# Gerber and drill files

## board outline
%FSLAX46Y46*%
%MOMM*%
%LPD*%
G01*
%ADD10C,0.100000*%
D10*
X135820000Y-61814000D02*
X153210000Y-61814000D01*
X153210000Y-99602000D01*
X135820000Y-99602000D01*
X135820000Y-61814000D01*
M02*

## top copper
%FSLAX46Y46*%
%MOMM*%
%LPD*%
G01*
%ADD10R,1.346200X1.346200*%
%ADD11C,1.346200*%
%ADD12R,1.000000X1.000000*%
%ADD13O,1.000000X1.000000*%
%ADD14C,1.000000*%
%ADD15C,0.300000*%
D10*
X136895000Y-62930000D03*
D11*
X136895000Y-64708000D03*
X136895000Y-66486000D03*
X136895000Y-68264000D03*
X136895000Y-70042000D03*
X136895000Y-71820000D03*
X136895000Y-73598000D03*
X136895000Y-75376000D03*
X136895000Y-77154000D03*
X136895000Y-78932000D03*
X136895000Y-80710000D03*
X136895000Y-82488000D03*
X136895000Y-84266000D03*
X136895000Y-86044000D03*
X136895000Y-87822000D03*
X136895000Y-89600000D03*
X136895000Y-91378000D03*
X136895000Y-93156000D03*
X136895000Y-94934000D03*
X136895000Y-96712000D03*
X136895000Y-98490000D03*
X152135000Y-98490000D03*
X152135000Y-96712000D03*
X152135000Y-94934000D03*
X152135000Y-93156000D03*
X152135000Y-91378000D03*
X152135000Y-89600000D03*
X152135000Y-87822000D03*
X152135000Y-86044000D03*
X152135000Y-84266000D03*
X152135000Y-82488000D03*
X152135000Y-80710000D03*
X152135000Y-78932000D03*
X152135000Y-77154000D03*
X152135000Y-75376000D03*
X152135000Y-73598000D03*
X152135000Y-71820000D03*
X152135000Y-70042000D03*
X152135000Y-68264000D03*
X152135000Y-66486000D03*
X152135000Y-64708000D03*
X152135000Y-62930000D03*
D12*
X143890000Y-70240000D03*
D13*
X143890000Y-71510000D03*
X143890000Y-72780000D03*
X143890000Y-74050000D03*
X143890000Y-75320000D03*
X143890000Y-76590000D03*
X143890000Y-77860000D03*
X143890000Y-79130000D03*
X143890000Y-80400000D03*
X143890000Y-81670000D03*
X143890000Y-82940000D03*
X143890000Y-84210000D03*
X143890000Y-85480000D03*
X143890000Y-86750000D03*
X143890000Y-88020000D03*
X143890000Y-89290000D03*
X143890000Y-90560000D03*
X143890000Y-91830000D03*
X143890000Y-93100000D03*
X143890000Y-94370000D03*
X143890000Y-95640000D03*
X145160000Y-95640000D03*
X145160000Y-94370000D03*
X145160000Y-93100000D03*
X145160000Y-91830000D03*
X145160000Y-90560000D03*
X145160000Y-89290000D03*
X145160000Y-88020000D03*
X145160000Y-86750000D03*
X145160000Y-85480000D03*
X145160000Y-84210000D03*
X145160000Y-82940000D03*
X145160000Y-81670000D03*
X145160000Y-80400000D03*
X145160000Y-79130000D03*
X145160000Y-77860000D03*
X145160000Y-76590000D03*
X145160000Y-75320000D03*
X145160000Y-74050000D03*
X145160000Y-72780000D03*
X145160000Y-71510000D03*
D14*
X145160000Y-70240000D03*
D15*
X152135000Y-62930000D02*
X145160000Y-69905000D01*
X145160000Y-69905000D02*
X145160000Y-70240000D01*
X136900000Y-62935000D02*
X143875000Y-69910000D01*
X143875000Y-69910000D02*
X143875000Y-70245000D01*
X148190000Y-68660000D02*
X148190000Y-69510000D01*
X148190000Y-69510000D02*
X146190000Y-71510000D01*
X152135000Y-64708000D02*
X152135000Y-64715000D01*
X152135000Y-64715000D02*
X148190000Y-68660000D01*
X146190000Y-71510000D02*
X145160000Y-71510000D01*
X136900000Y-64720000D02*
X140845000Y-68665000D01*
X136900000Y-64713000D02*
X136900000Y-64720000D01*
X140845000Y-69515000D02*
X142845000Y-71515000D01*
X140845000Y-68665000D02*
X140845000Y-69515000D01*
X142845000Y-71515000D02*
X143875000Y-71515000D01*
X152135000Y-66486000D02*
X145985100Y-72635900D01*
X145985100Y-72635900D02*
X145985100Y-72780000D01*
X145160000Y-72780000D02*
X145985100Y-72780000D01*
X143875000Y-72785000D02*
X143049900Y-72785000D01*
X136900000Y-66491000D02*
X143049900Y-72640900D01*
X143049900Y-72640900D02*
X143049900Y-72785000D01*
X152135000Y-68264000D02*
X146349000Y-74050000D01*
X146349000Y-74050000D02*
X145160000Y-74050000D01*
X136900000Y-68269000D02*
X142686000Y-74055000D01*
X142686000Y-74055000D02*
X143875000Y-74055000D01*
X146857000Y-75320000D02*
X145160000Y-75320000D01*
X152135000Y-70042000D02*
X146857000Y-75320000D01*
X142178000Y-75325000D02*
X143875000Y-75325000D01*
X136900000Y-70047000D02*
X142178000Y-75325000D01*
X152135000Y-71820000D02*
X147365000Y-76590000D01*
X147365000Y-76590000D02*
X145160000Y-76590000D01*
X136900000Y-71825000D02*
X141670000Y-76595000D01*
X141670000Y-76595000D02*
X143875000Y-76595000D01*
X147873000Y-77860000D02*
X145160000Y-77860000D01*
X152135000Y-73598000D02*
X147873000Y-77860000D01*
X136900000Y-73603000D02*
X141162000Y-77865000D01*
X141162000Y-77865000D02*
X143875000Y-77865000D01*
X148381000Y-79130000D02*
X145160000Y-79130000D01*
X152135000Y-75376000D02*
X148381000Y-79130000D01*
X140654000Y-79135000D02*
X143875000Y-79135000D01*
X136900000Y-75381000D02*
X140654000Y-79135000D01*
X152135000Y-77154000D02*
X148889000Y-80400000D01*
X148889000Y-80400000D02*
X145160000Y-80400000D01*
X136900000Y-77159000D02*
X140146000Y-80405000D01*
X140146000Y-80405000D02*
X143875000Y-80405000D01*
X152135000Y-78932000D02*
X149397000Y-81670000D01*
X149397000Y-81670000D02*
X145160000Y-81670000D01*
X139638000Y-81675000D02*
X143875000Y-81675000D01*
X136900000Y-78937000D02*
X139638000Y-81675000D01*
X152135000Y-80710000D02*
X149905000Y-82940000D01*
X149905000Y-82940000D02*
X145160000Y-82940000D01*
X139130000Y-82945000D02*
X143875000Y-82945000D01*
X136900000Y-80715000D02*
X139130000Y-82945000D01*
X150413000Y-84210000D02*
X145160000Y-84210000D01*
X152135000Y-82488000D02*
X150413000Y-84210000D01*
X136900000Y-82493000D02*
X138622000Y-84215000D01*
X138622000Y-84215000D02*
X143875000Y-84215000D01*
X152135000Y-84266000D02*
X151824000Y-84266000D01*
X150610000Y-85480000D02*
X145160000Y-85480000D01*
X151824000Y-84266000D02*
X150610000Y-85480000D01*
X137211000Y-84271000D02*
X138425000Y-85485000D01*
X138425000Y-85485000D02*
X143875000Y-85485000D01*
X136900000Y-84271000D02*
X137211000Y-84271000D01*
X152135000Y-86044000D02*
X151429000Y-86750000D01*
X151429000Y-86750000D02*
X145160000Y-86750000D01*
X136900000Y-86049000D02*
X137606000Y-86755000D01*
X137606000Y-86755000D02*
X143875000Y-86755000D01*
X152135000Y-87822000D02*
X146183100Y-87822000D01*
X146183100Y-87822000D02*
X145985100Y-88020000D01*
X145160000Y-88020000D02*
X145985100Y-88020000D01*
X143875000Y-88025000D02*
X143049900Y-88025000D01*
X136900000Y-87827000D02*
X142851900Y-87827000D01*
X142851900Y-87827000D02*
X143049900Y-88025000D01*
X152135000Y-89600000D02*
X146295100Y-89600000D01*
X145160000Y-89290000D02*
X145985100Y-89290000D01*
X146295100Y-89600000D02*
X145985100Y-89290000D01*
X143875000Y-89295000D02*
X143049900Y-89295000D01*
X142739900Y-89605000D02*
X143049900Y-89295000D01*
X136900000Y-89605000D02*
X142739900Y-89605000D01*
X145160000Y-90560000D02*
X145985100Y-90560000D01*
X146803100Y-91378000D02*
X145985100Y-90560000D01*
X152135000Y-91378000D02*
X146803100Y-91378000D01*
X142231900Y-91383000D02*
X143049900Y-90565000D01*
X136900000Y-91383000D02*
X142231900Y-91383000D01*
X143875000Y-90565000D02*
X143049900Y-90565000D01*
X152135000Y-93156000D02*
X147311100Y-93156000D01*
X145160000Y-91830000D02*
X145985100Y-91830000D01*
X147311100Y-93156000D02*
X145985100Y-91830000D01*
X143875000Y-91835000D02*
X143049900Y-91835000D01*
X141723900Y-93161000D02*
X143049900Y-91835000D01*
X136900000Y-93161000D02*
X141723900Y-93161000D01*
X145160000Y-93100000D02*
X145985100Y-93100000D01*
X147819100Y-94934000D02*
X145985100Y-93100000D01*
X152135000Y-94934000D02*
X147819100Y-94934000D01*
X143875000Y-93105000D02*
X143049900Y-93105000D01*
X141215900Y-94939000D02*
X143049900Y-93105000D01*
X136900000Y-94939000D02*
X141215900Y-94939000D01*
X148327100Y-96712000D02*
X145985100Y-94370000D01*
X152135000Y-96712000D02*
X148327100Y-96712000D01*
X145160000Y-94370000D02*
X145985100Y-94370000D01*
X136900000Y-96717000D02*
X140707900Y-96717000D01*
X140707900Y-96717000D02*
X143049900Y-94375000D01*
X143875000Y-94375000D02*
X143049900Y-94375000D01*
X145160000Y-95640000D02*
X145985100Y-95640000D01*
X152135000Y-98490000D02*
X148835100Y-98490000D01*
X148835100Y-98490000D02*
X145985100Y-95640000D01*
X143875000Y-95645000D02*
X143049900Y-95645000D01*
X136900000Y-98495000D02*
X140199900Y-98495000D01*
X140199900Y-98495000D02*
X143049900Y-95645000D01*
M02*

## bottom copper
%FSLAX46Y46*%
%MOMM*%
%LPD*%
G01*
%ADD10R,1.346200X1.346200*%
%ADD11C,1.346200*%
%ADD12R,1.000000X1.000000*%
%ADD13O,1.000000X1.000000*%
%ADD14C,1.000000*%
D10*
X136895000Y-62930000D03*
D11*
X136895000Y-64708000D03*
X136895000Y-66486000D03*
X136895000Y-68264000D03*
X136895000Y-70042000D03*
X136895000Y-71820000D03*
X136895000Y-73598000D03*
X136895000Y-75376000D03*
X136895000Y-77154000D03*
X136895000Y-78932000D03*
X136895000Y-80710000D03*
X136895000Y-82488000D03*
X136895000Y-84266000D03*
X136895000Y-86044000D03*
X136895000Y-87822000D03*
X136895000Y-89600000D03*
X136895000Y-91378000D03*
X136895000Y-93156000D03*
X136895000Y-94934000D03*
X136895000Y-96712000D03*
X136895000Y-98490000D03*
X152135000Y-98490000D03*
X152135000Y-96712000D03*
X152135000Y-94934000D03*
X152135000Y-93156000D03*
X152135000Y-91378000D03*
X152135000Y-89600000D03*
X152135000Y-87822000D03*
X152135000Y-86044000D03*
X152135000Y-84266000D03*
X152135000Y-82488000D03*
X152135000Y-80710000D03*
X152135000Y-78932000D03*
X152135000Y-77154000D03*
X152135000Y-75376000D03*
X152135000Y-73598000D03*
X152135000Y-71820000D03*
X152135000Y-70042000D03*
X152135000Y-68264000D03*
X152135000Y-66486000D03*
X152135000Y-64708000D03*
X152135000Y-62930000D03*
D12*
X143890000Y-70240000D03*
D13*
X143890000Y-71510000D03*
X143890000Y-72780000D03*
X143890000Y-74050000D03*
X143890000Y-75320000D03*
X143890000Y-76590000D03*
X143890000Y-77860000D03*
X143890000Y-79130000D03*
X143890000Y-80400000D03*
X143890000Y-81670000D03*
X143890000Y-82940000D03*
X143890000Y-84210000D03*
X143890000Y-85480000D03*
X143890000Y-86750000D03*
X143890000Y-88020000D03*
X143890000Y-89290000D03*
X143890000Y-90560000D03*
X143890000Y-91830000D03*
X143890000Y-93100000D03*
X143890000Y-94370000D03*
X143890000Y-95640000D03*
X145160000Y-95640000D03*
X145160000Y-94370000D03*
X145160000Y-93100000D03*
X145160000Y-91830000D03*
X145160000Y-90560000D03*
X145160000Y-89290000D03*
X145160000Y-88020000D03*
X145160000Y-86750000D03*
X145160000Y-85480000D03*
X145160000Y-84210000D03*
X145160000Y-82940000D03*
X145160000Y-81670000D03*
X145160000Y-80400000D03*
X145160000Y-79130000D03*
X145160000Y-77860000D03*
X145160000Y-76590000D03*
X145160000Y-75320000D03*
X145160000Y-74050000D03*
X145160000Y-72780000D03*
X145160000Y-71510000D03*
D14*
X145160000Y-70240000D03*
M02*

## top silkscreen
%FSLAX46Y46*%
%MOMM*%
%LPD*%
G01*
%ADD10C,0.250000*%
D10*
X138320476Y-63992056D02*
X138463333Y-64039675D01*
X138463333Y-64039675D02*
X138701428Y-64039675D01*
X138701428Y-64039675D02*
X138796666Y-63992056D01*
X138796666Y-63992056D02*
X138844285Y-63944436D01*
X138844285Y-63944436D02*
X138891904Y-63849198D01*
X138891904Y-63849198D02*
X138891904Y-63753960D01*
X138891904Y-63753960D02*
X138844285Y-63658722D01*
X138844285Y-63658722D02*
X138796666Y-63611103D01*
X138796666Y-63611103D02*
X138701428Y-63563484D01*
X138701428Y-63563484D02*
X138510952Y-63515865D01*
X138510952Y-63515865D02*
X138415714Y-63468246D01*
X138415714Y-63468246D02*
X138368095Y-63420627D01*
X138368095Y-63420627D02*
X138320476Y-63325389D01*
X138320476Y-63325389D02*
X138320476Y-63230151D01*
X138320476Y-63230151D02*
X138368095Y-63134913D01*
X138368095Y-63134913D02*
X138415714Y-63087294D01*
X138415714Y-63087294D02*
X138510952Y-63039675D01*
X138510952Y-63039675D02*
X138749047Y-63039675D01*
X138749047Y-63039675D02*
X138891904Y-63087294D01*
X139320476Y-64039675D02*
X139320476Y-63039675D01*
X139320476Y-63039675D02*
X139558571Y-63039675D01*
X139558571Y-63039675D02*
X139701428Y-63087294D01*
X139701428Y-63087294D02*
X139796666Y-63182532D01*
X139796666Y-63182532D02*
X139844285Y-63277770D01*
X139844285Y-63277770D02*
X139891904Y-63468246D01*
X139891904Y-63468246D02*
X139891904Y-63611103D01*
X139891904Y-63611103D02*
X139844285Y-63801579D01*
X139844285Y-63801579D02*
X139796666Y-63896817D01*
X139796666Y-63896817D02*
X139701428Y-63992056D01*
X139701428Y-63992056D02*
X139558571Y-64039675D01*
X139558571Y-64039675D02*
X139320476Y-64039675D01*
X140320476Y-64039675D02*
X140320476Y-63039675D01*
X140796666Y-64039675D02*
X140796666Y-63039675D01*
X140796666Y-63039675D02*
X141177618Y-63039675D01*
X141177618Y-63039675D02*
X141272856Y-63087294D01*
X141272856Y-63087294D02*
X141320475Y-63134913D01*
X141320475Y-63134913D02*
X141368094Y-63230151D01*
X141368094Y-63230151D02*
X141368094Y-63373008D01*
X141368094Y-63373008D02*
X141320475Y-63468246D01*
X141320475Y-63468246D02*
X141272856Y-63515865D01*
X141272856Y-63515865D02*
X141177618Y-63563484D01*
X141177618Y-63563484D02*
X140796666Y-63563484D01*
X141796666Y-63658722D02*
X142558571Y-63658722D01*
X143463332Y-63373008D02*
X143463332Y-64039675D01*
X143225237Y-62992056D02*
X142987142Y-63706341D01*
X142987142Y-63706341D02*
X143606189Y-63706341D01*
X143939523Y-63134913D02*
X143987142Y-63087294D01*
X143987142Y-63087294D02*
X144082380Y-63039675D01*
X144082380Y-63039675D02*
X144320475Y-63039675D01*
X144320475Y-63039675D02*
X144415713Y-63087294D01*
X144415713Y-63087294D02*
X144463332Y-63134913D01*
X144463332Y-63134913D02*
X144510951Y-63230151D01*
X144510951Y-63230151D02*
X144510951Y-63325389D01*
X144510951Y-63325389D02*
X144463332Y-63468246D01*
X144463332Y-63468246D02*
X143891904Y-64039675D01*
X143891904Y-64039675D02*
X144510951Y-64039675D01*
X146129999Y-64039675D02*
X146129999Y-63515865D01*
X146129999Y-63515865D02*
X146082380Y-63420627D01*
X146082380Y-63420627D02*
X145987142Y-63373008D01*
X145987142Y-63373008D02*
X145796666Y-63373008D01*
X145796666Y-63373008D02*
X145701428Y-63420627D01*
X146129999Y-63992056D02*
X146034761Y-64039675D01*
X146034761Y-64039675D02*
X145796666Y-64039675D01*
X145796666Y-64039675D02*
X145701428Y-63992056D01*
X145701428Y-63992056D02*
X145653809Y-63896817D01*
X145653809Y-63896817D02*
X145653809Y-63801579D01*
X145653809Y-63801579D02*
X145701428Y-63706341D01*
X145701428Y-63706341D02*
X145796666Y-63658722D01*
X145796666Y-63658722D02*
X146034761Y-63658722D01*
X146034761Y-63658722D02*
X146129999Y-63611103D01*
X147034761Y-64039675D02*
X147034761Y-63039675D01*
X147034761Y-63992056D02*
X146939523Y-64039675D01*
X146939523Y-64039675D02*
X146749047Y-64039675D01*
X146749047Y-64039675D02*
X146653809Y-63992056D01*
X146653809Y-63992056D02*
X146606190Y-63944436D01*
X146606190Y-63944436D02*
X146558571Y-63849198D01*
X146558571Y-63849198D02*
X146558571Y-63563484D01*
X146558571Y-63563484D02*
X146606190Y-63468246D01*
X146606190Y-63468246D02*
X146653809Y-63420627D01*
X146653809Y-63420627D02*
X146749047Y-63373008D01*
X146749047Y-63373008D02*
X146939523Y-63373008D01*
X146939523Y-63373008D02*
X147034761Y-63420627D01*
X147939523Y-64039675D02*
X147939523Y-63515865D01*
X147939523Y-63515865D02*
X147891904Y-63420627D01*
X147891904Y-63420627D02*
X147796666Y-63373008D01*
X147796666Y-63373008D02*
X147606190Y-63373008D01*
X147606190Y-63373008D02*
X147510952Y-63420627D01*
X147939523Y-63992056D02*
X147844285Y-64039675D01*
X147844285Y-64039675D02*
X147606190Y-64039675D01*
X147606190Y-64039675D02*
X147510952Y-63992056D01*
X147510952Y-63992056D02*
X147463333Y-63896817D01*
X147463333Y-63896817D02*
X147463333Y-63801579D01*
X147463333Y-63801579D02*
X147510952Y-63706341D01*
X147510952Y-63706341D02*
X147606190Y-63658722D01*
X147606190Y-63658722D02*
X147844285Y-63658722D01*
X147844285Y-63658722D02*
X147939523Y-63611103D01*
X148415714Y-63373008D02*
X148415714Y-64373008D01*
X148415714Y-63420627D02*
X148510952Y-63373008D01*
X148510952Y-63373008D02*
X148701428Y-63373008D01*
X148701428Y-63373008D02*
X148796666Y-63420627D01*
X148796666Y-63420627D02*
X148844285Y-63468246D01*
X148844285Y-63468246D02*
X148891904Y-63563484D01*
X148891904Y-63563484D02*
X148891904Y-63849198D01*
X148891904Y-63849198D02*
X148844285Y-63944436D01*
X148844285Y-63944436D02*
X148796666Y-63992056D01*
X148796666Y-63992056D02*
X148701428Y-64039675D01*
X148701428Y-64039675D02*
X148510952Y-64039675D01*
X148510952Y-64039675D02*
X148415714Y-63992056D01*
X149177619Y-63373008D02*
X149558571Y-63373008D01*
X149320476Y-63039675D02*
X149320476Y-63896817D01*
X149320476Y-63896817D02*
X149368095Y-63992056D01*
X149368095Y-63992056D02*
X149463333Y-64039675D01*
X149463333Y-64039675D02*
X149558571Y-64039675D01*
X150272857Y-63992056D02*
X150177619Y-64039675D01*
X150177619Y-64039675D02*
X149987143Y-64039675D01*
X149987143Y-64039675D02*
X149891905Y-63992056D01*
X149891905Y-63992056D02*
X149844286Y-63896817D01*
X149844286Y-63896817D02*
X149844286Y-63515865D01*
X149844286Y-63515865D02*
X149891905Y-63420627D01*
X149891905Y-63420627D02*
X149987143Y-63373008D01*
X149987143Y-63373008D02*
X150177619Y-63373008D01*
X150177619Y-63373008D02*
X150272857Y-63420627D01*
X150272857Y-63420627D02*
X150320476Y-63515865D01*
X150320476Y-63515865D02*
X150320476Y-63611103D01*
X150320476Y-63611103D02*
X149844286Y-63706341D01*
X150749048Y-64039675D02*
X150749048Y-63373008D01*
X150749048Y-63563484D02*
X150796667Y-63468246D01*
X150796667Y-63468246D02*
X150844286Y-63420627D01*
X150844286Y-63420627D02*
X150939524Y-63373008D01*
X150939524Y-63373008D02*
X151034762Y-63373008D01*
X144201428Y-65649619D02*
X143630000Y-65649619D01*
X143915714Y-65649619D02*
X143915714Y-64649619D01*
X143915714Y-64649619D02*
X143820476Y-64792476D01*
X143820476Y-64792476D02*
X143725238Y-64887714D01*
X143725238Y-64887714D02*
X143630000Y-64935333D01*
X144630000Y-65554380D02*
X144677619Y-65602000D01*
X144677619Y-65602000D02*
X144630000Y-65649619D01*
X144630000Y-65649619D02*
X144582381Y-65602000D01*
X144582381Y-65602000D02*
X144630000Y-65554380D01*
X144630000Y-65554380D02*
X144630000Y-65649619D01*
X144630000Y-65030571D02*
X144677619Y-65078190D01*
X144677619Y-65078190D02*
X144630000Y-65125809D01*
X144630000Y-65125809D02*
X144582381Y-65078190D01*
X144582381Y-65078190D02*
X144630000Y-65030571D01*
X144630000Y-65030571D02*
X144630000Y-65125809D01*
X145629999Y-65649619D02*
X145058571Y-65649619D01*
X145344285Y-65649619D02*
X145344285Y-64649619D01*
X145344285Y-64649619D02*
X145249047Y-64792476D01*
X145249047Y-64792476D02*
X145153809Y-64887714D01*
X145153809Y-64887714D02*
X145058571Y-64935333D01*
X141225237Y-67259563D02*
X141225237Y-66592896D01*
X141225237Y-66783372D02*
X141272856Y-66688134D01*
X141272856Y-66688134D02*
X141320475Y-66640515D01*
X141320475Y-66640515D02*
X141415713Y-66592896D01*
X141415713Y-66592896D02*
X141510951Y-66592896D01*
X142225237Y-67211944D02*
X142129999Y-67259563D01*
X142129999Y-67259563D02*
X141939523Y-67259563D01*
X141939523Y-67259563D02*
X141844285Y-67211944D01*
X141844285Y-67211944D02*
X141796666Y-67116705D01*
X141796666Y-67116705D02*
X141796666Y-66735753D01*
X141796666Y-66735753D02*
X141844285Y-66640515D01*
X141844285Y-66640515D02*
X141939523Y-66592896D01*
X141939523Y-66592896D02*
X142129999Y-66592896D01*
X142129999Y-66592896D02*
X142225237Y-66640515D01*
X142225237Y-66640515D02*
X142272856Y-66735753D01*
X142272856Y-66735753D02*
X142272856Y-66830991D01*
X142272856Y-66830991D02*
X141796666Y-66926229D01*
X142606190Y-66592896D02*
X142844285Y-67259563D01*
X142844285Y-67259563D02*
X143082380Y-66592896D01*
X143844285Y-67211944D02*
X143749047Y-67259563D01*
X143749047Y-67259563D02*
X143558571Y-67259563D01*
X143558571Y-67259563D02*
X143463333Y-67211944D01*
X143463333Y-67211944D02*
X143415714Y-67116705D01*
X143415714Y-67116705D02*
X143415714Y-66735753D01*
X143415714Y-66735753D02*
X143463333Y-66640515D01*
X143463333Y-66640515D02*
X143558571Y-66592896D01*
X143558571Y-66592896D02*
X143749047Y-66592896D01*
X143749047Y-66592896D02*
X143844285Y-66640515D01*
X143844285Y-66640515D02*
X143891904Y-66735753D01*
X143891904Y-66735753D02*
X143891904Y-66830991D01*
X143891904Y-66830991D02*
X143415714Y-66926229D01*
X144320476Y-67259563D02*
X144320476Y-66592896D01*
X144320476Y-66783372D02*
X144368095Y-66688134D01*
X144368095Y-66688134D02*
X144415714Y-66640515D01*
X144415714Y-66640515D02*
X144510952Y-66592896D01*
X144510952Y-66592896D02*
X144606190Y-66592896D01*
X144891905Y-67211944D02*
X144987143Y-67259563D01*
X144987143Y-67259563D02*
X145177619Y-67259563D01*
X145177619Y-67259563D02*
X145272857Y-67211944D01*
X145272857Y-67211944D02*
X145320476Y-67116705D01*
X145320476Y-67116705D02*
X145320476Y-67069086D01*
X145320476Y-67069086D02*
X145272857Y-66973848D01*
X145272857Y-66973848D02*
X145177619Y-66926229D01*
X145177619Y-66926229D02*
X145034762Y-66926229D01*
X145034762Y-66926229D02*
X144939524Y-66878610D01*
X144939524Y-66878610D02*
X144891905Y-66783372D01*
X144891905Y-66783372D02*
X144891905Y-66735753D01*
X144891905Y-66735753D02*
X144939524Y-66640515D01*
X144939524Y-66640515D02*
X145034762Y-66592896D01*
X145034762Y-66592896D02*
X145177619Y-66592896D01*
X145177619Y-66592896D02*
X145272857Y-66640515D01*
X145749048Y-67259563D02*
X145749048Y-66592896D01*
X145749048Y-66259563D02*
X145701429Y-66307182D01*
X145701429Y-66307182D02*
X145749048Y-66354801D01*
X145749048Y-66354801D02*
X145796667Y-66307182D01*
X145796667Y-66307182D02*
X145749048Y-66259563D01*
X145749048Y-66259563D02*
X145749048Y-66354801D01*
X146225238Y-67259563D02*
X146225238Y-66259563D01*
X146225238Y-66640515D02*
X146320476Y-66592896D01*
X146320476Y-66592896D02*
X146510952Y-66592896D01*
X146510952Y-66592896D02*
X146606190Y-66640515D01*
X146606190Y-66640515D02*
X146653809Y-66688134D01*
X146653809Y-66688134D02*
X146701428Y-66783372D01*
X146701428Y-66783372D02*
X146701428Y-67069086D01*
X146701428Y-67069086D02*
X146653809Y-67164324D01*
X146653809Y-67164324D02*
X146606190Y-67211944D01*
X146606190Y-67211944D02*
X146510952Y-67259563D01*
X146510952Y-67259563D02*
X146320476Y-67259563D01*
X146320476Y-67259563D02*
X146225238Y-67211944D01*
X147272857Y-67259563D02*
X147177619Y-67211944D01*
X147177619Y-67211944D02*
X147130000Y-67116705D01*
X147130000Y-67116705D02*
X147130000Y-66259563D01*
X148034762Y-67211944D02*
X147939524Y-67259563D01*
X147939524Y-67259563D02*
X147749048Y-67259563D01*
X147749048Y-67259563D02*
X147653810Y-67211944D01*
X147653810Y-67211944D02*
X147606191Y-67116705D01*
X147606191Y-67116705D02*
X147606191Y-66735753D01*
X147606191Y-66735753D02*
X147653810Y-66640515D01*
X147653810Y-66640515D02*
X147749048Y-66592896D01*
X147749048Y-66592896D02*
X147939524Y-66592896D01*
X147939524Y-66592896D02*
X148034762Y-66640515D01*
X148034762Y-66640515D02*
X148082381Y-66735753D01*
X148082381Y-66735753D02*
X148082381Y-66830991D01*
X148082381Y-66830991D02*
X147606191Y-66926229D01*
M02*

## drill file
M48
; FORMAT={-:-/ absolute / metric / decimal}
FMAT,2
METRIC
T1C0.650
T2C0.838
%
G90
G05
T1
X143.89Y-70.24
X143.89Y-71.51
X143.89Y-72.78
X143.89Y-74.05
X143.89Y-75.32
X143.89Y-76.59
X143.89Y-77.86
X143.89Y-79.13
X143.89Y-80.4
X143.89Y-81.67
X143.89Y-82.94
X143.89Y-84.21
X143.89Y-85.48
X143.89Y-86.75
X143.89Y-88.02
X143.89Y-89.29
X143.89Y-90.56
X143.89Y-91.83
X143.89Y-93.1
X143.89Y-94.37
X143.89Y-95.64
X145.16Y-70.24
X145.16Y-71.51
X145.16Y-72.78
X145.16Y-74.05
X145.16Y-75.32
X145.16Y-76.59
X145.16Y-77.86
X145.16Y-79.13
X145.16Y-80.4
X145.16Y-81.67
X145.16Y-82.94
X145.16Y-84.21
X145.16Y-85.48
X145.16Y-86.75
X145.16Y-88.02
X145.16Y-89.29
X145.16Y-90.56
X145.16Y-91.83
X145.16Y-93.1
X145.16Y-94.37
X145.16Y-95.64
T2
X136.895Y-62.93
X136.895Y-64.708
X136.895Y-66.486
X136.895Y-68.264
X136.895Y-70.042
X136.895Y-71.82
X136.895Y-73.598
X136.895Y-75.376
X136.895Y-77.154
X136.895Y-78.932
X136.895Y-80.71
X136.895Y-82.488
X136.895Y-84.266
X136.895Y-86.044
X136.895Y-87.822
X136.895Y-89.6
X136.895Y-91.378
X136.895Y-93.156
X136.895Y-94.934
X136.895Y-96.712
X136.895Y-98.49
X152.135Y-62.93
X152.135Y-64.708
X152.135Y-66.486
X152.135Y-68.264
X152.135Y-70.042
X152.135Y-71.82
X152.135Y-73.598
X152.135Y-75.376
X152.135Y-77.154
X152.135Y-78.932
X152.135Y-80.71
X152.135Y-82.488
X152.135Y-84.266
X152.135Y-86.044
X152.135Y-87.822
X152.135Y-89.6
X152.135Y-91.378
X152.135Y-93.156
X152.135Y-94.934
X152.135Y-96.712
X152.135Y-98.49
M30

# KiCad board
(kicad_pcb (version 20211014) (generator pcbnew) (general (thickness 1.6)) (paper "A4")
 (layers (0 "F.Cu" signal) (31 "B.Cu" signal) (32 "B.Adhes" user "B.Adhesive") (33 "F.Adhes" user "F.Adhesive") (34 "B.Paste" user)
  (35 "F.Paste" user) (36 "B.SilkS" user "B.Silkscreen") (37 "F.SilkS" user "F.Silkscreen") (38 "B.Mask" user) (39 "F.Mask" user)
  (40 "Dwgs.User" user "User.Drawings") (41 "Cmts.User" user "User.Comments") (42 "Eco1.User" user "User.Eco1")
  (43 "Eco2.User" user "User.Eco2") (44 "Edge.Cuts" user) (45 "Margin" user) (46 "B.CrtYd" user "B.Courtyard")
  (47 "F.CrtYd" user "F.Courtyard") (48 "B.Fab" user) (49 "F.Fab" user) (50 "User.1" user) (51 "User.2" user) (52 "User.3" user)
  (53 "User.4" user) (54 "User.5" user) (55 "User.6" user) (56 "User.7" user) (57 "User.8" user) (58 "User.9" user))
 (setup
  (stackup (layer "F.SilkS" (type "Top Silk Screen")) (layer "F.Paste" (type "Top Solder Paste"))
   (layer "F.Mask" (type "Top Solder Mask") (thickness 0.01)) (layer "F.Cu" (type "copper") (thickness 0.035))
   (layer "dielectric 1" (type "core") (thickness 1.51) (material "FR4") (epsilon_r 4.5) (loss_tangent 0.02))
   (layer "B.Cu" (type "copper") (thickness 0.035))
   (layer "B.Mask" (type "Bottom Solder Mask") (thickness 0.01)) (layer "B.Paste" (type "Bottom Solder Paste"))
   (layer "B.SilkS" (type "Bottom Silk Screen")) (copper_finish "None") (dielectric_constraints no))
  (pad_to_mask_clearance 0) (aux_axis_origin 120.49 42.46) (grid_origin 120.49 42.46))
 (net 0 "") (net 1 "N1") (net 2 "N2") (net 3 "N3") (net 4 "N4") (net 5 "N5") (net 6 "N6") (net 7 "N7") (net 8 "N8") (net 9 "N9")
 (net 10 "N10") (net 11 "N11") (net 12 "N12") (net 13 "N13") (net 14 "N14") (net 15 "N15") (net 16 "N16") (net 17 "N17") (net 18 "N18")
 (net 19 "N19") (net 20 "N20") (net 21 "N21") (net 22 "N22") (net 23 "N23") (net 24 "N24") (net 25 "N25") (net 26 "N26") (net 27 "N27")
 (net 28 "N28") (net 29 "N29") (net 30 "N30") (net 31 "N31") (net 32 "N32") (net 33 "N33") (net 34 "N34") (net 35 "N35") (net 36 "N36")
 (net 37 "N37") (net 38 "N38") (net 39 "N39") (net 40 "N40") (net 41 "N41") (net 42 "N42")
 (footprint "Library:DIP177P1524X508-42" (layer "F.Cu") (at 152.135 98.49)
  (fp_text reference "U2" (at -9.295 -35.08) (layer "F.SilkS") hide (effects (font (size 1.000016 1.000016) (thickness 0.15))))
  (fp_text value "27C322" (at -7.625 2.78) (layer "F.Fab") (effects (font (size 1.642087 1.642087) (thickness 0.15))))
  (pad "1" thru_hole rect (at -15.24 -35.56) (size 1.3462 1.3462) (drill 0.8382) (layers *.Cu *.Mask) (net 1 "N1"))
  (pad "2" thru_hole circle (at -15.24 -33.782) (size 1.3462 1.3462) (drill 0.8382) (layers *.Cu *.Mask) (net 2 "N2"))
  (pad "3" thru_hole circle (at -15.24 -32.004) (size 1.3462 1.3462) (drill 0.8382) (layers *.Cu *.Mask) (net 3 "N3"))
  (pad "4" thru_hole circle (at -15.24 -30.226) (size 1.3462 1.3462) (drill 0.8382) (layers *.Cu *.Mask) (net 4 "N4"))
  (pad "5" thru_hole circle (at -15.24 -28.448) (size 1.3462 1.3462) (drill 0.8382) (layers *.Cu *.Mask) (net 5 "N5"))
  (pad "6" thru_hole circle (at -15.24 -26.67) (size 1.3462 1.3462) (drill 0.8382) (layers *.Cu *.Mask) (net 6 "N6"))
  (pad "7" thru_hole circle (at -15.24 -24.892) (size 1.3462 1.3462) (drill 0.8382) (layers *.Cu *.Mask) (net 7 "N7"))
  (pad "8" thru_hole circle (at -15.24 -23.114) (size 1.3462 1.3462) (drill 0.8382) (layers *.Cu *.Mask) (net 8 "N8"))
  (pad "9" thru_hole circle (at -15.24 -21.336) (size 1.3462 1.3462) (drill 0.8382) (layers *.Cu *.Mask) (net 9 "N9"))
  (pad "10" thru_hole circle (at -15.24 -19.558) (size 1.3462 1.3462) (drill 0.8382) (layers *.Cu *.Mask) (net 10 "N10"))
  (pad "11" thru_hole circle (at -15.24 -17.78) (size 1.3462 1.3462) (drill 0.8382) (layers *.Cu *.Mask) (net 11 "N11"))
  (pad "12" thru_hole circle (at -15.24 -16.002) (size 1.3462 1.3462) (drill 0.8382) (layers *.Cu *.Mask) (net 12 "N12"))
  (pad "13" thru_hole circle (at -15.24 -14.224) (size 1.3462 1.3462) (drill 0.8382) (layers *.Cu *.Mask) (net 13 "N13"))
  (pad "14" thru_hole circle (at -15.24 -12.446) (size 1.3462 1.3462) (drill 0.8382) (layers *.Cu *.Mask) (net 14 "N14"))
  (pad "15" thru_hole circle (at -15.24 -10.668) (size 1.3462 1.3462) (drill 0.8382) (layers *.Cu *.Mask) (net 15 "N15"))
  (pad "16" thru_hole circle (at -15.24 -8.89) (size 1.3462 1.3462) (drill 0.8382) (layers *.Cu *.Mask) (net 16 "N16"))
  (pad "17" thru_hole circle (at -15.24 -7.112) (size 1.3462 1.3462) (drill 0.8382) (layers *.Cu *.Mask) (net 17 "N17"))
  (pad "18" thru_hole circle (at -15.24 -5.334) (size 1.3462 1.3462) (drill 0.8382) (layers *.Cu *.Mask) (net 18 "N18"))
  (pad "19" thru_hole circle (at -15.24 -3.556) (size 1.3462 1.3462) (drill 0.8382) (layers *.Cu *.Mask) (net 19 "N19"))
  (pad "20" thru_hole circle (at -15.24 -1.778) (size 1.3462 1.3462) (drill 0.8382) (layers *.Cu *.Mask) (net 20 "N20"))
  (pad "21" thru_hole circle (at -15.24 0) (size 1.3462 1.3462) (drill 0.8382) (layers *.Cu *.Mask) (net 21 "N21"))
  (pad "22" thru_hole circle (at 0 0) (size 1.3462 1.3462) (drill 0.8382) (layers *.Cu *.Mask) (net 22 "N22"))
  (pad "23" thru_hole circle (at 0 -1.778) (size 1.3462 1.3462) (drill 0.8382) (layers *.Cu *.Mask) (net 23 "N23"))
  (pad "24" thru_hole circle (at 0 -3.556) (size 1.3462 1.3462) (drill 0.8382) (layers *.Cu *.Mask) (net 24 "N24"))
  (pad "25" thru_hole circle (at 0 -5.334) (size 1.3462 1.3462) (drill 0.8382) (layers *.Cu *.Mask) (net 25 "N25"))
  (pad "26" thru_hole circle (at 0 -7.112) (size 1.3462 1.3462) (drill 0.8382) (layers *.Cu *.Mask) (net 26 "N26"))
  (pad "27" thru_hole circle (at 0 -8.89) (size 1.3462 1.3462) (drill 0.8382) (layers *.Cu *.Mask) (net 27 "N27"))
  (pad "28" thru_hole circle (at 0 -10.668) (size 1.3462 1.3462) (drill 0.8382) (layers *.Cu *.Mask) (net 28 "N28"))
  (pad "29" thru_hole circle (at 0 -12.446) (size 1.3462 1.3462) (drill 0.8382) (layers *.Cu *.Mask) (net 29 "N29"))
  (pad "30" thru_hole circle (at 0 -14.224) (size 1.3462 1.3462) (drill 0.8382) (layers *.Cu *.Mask) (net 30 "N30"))
  (pad "31" thru_hole circle (at 0 -16.002) (size 1.3462 1.3462) (drill 0.8382) (layers *.Cu *.Mask) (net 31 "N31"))
  (pad "32" thru_hole circle (at 0 -17.78) (size 1.3462 1.3462) (drill 0.8382) (layers *.Cu *.Mask) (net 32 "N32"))
  (pad "33" thru_hole circle (at 0 -19.558) (size 1.3462 1.3462) (drill 0.8382) (layers *.Cu *.Mask) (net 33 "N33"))
  (pad "34" thru_hole circle (at 0 -21.336) (size 1.3462 1.3462) (drill 0.8382) (layers *.Cu *.Mask) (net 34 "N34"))
  (pad "35" thru_hole circle (at 0 -23.114) (size 1.3462 1.3462) (drill 0.8382) (layers *.Cu *.Mask) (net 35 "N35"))
  (pad "36" thru_hole circle (at 0 -24.892) (size 1.3462 1.3462) (drill 0.8382) (layers *.Cu *.Mask) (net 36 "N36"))
  (pad "37" thru_hole circle (at 0 -26.67) (size 1.3462 1.3462) (drill 0.8382) (layers *.Cu *.Mask) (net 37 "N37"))
  (pad "38" thru_hole circle (at 0 -28.448) (size 1.3462 1.3462) (drill 0.8382) (layers *.Cu *.Mask) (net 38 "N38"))
  (pad "39" thru_hole circle (at 0 -30.226) (size 1.3462 1.3462) (drill 0.8382) (layers *.Cu *.Mask) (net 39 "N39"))
  (pad "40" thru_hole circle (at 0 -32.004) (size 1.3462 1.3462) (drill 0.8382) (layers *.Cu *.Mask) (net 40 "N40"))
  (pad "41" thru_hole circle (at 0 -33.782) (size 1.3462 1.3462) (drill 0.8382) (layers *.Cu *.Mask) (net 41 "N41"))
  (pad "42" thru_hole circle (at 0 -35.56) (size 1.3462 1.3462) (drill 0.8382) (layers *.Cu *.Mask) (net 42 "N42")))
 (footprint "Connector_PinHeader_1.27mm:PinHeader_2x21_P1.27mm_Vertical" (layer "B.Cu") (at 145.16 70.24 180)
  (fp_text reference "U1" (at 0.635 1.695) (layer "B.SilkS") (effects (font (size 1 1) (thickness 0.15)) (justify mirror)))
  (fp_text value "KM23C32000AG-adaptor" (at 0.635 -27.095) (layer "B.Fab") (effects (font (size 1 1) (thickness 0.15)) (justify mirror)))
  (pad "1" thru_hole rect (at 1.27 0 180) (size 1 1) (drill 0.65) (layers *.Cu *.Mask) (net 1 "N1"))
  (pad "2" thru_hole oval (at 1.27 -1.27 180) (size 1 1) (drill 0.65) (layers *.Cu *.Mask) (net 2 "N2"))
  (pad "3" thru_hole oval (at 1.27 -2.54 180) (size 1 1) (drill 0.65) (layers *.Cu *.Mask) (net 3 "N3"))
  (pad "4" thru_hole oval (at 1.27 -3.81 180) (size 1 1) (drill 0.65) (layers *.Cu *.Mask) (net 4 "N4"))
  (pad "5" thru_hole oval (at 1.27 -5.08 180) (size 1 1) (drill 0.65) (layers *.Cu *.Mask) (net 5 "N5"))
  (pad "6" thru_hole oval (at 1.27 -6.35 180) (size 1 1) (drill 0.65) (layers *.Cu *.Mask) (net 6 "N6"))
  (pad "7" thru_hole oval (at 1.27 -7.62 180) (size 1 1) (drill 0.65) (layers *.Cu *.Mask) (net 7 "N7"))
  (pad "8" thru_hole oval (at 1.27 -8.89 180) (size 1 1) (drill 0.65) (layers *.Cu *.Mask) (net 8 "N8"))
  (pad "9" thru_hole oval (at 1.27 -10.16 180) (size 1 1) (drill 0.65) (layers *.Cu *.Mask) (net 9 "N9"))
  (pad "10" thru_hole oval (at 1.27 -11.43 180) (size 1 1) (drill 0.65) (layers *.Cu *.Mask) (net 10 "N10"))
  (pad "11" thru_hole oval (at 1.27 -12.7 180) (size 1 1) (drill 0.65) (layers *.Cu *.Mask) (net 11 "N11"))
  (pad "12" thru_hole oval (at 1.27 -13.97 180) (size 1 1) (drill 0.65) (layers *.Cu *.Mask) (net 12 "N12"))
  (pad "13" thru_hole oval (at 1.27 -15.24 180) (size 1 1) (drill 0.65) (layers *.Cu *.Mask) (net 13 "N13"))
  (pad "14" thru_hole oval (at 1.27 -16.51 180) (size 1 1) (drill 0.65) (layers *.Cu *.Mask) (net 14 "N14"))
  (pad "15" thru_hole oval (at 1.27 -17.78 180) (size 1 1) (drill 0.65) (layers *.Cu *.Mask) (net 15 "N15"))
  (pad "16" thru_hole oval (at 1.27 -19.05 180) (size 1 1) (drill 0.65) (layers *.Cu *.Mask) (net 16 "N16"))
  (pad "17" thru_hole oval (at 1.27 -20.32 180) (size 1 1) (drill 0.65) (layers *.Cu *.Mask) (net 17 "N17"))
  (pad "18" thru_hole oval (at 1.27 -21.59 180) (size 1 1) (drill 0.65) (layers *.Cu *.Mask) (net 18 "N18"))
  (pad "19" thru_hole oval (at 1.27 -22.86 180) (size 1 1) (drill 0.65) (layers *.Cu *.Mask) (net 19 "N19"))
  (pad "20" thru_hole oval (at 1.27 -24.13 180) (size 1 1) (drill 0.65) (layers *.Cu *.Mask) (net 20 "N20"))
  (pad "21" thru_hole oval (at 1.27 -25.4 180) (size 1 1) (drill 0.65) (layers *.Cu *.Mask) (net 21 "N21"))
  (pad "22" thru_hole oval (at 0 -25.4 180) (size 1 1) (drill 0.65) (layers *.Cu *.Mask) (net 22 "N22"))
  (pad "23" thru_hole oval (at 0 -24.13 180) (size 1 1) (drill 0.65) (layers *.Cu *.Mask) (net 23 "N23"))
  (pad "24" thru_hole oval (at 0 -22.86 180) (size 1 1) (drill 0.65) (layers *.Cu *.Mask) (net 24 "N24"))
  (pad "25" thru_hole oval (at 0 -21.59 180) (size 1 1) (drill 0.65) (layers *.Cu *.Mask) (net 25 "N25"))
  (pad "26" thru_hole oval (at 0 -20.32 180) (size 1 1) (drill 0.65) (layers *.Cu *.Mask) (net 26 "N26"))
  (pad "27" thru_hole oval (at 0 -19.05 180) (size 1 1) (drill 0.65) (layers *.Cu *.Mask) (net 27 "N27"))
  (pad "28" thru_hole oval (at 0 -17.78 180) (size 1 1) (drill 0.65) (layers *.Cu *.Mask) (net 28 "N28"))
  (pad "29" thru_hole oval (at 0 -16.51 180) (size 1 1) (drill 0.65) (layers *.Cu *.Mask) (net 29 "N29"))
  (pad "30" thru_hole oval (at 0 -15.24 180) (size 1 1) (drill 0.65) (layers *.Cu *.Mask) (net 30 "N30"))
  (pad "31" thru_hole oval (at 0 -13.97 180) (size 1 1) (drill 0.65) (layers *.Cu *.Mask) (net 31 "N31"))
  (pad "32" thru_hole oval (at 0 -12.7 180) (size 1 1) (drill 0.65) (layers *.Cu *.Mask) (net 32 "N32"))
  (pad "33" thru_hole oval (at 0 -11.43 180) (size 1 1) (drill 0.65) (layers *.Cu *.Mask) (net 33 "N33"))
  (pad "34" thru_hole oval (at 0 -10.16 180) (size 1 1) (drill 0.65) (layers *.Cu *.Mask) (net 34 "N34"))
  (pad "35" thru_hole oval (at 0 -8.89 180) (size 1 1) (drill 0.65) (layers *.Cu *.Mask) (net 35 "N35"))
  (pad "36" thru_hole oval (at 0 -7.62 180) (size 1 1) (drill 0.65) (layers *.Cu *.Mask) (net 36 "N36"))
  (pad "37" thru_hole oval (at 0 -6.35 180) (size 1 1) (drill 0.65) (layers *.Cu *.Mask) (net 37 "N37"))
  (pad "38" thru_hole oval (at 0 -5.08 180) (size 1 1) (drill 0.65) (layers *.Cu *.Mask) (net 38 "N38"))
  (pad "39" thru_hole oval (at 0 -3.81 180) (size 1 1) (drill 0.65) (layers *.Cu *.Mask) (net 39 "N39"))
  (pad "40" thru_hole oval (at 0 -2.54 180) (size 1 1) (drill 0.65) (layers *.Cu *.Mask) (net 40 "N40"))
  (pad "41" thru_hole oval (at 0 -1.27 180) (size 1 1) (drill 0.65) (layers *.Cu *.Mask) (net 41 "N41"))
  (pad "42" thru_hole circle (at 0 0 180) (size 1 1) (drill 0.65) (layers *.Cu *.Mask) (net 42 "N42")))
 (gr_rect (start 135.82 61.814) (end 153.21 99.602) (layer "Edge.Cuts") (width 0.1) (fill none))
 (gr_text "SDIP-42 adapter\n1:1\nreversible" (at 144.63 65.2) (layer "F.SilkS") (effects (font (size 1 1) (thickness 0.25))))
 (segment (start 152.135 62.93) (end 145.16 69.905) (width 0.3) (layer "F.Cu") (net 42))
 (segment (start 145.16 69.905) (end 145.16 70.24) (width 0.3) (layer "F.Cu") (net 42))
 (segment (start 136.9 62.935) (end 143.875 69.91) (width 0.3) (layer "F.Cu") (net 1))
 (segment (start 143.875 69.91) (end 143.875 70.245) (width 0.3) (layer "F.Cu") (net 1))
 (segment (start 148.19 68.66) (end 148.19 69.51) (width 0.3) (layer "F.Cu") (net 41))
 (segment (start 148.19 69.51) (end 146.19 71.51) (width 0.3) (layer "F.Cu") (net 41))
 (segment (start 152.135 64.708) (end 152.135 64.715) (width 0.3) (layer "F.Cu") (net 41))
 (segment (start 152.135 64.715) (end 148.19 68.66) (width 0.3) (layer "F.Cu") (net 41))
 (segment (start 146.19 71.51) (end 145.16 71.51) (width 0.3) (layer "F.Cu") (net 41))
 (segment (start 136.9 64.72) (end 140.845 68.665) (width 0.3) (layer "F.Cu") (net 2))
 (segment (start 136.9 64.713) (end 136.9 64.72) (width 0.3) (layer "F.Cu") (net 2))
 (segment (start 140.845 69.515) (end 142.845 71.515) (width 0.3) (layer "F.Cu") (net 2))
 (segment (start 140.845 68.665) (end 140.845 69.515) (width 0.3) (layer "F.Cu") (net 2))
 (segment (start 142.845 71.515) (end 143.875 71.515) (width 0.3) (layer "F.Cu") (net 2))
 (segment (start 152.135 66.486) (end 145.9851 72.6359) (width 0.3) (layer "F.Cu") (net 40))
 (segment (start 145.9851 72.6359) (end 145.9851 72.78) (width 0.3) (layer "F.Cu") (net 40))
 (segment (start 145.16 72.78) (end 145.9851 72.78) (width 0.3) (layer "F.Cu") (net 40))
 (segment (start 143.875 72.785) (end 143.0499 72.785) (width 0.3) (layer "F.Cu") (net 3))
 (segment (start 136.9 66.491) (end 143.0499 72.6409) (width 0.3) (layer "F.Cu") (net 3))
 (segment (start 143.0499 72.6409) (end 143.0499 72.785) (width 0.3) (layer "F.Cu") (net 3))
 (segment (start 152.135 68.264) (end 146.349 74.05) (width 0.3) (layer "F.Cu") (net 39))
 (segment (start 146.349 74.05) (end 145.16 74.05) (width 0.3) (layer "F.Cu") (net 39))
 (segment (start 136.9 68.269) (end 142.686 74.055) (width 0.3) (layer "F.Cu") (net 4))
 (segment (start 142.686 74.055) (end 143.875 74.055) (width 0.3) (layer "F.Cu") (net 4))
 (segment (start 146.857 75.32) (end 145.16 75.32) (width 0.3) (layer "F.Cu") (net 38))
 (segment (start 152.135 70.042) (end 146.857 75.32) (width 0.3) (layer "F.Cu") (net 38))
 (segment (start 142.178 75.325) (end 143.875 75.325) (width 0.3) (layer "F.Cu") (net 5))
 (segment (start 136.9 70.047) (end 142.178 75.325) (width 0.3) (layer "F.Cu") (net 5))
 (segment (start 152.135 71.82) (end 147.365 76.59) (width 0.3) (layer "F.Cu") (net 37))
 (segment (start 147.365 76.59) (end 145.16 76.59) (width 0.3) (layer "F.Cu") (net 37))
 (segment (start 136.9 71.825) (end 141.67 76.595) (width 0.3) (layer "F.Cu") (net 6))
 (segment (start 141.67 76.595) (end 143.875 76.595) (width 0.3) (layer "F.Cu") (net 6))
 (segment (start 147.873 77.86) (end 145.16 77.86) (width 0.3) (layer "F.Cu") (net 36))
 (segment (start 152.135 73.598) (end 147.873 77.86) (width 0.3) (layer "F.Cu") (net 36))
 (segment (start 136.9 73.603) (end 141.162 77.865) (width 0.3) (layer "F.Cu") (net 7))
 (segment (start 141.162 77.865) (end 143.875 77.865) (width 0.3) (layer "F.Cu") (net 7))
 (segment (start 148.381 79.13) (end 145.16 79.13) (width 0.3) (layer "F.Cu") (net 35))
 (segment (start 152.135 75.376) (end 148.381 79.13) (width 0.3) (layer "F.Cu") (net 35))
 (segment (start 140.654 79.135) (end 143.875 79.135) (width 0.3) (layer "F.Cu") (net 8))
 (segment (start 136.9 75.381) (end 140.654 79.135) (width 0.3) (layer "F.Cu") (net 8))
 (segment (start 152.135 77.154) (end 148.889 80.4) (width 0.3) (layer "F.Cu") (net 34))
 (segment (start 148.889 80.4) (end 145.16 80.4) (width 0.3) (layer "F.Cu") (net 34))
 (segment (start 136.9 77.159) (end 140.146 80.405) (width 0.3) (layer "F.Cu") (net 9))
 (segment (start 140.146 80.405) (end 143.875 80.405) (width 0.3) (layer "F.Cu") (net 9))
 (segment (start 152.135 78.932) (end 149.397 81.67) (width 0.3) (layer "F.Cu") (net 33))
 (segment (start 149.397 81.67) (end 145.16 81.67) (width 0.3) (layer "F.Cu") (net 33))
 (segment (start 139.638 81.675) (end 143.875 81.675) (width 0.3) (layer "F.Cu") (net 10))
 (segment (start 136.9 78.937) (end 139.638 81.675) (width 0.3) (layer "F.Cu") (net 10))
 (segment (start 152.135 80.71) (end 149.905 82.94) (width 0.3) (layer "F.Cu") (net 32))
 (segment (start 149.905 82.94) (end 145.16 82.94) (width 0.3) (layer "F.Cu") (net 32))
 (segment (start 139.13 82.945) (end 143.875 82.945) (width 0.3) (layer "F.Cu") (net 11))
 (segment (start 136.9 80.715) (end 139.13 82.945) (width 0.3) (layer "F.Cu") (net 11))
 (segment (start 150.413 84.21) (end 145.16 84.21) (width 0.3) (layer "F.Cu") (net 31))
 (segment (start 152.135 82.488) (end 150.413 84.21) (width 0.3) (layer "F.Cu") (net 31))
 (segment (start 136.9 82.493) (end 138.622 84.215) (width 0.3) (layer "F.Cu") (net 12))
 (segment (start 138.622 84.215) (end 143.875 84.215) (width 0.3) (layer "F.Cu") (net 12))
 (segment (start 152.135 84.266) (end 151.824 84.266) (width 0.3) (layer "F.Cu") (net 30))
 (segment (start 150.61 85.48) (end 145.16 85.48) (width 0.3) (layer "F.Cu") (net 30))
 (segment (start 151.824 84.266) (end 150.61 85.48) (width 0.3) (layer "F.Cu") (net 30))
 (segment (start 137.211 84.271) (end 138.425 85.485) (width 0.3) (layer "F.Cu") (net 13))
 (segment (start 138.425 85.485) (end 143.875 85.485) (width 0.3) (layer "F.Cu") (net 13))
 (segment (start 136.9 84.271) (end 137.211 84.271) (width 0.3) (layer "F.Cu") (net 13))
 (segment (start 152.135 86.044) (end 151.429 86.75) (width 0.3) (layer "F.Cu") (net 29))
 (segment (start 151.429 86.75) (end 145.16 86.75) (width 0.3) (layer "F.Cu") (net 29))
 (segment (start 136.9 86.049) (end 137.606 86.755) (width 0.3) (layer "F.Cu") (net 14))
 (segment (start 137.606 86.755) (end 143.875 86.755) (width 0.3) (layer "F.Cu") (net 14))
 (segment (start 152.135 87.822) (end 146.1831 87.822) (width 0.3) (layer "F.Cu") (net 28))
 (segment (start 146.1831 87.822) (end 145.9851 88.02) (width 0.3) (layer "F.Cu") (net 28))
 (segment (start 145.16 88.02) (end 145.9851 88.02) (width 0.3) (layer "F.Cu") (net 28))
 (segment (start 143.875 88.025) (end 143.0499 88.025) (width 0.3) (layer "F.Cu") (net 15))
 (segment (start 136.9 87.827) (end 142.8519 87.827) (width 0.3) (layer "F.Cu") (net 15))
 (segment (start 142.8519 87.827) (end 143.0499 88.025) (width 0.3) (layer "F.Cu") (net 15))
 (segment (start 152.135 89.6) (end 146.2951 89.6) (width 0.3) (layer "F.Cu") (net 27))
 (segment (start 145.16 89.29) (end 145.9851 89.29) (width 0.3) (layer "F.Cu") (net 27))
 (segment (start 146.2951 89.6) (end 145.9851 89.29) (width 0.3) (layer "F.Cu") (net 27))
 (segment (start 143.875 89.295) (end 143.0499 89.295) (width 0.3) (layer "F.Cu") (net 16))
 (segment (start 142.7399 89.605) (end 143.0499 89.295) (width 0.3) (layer "F.Cu") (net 16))
 (segment (start 136.9 89.605) (end 142.7399 89.605) (width 0.3) (layer "F.Cu") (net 16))
 (segment (start 145.16 90.56) (end 145.9851 90.56) (width 0.3) (layer "F.Cu") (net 26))
 (segment (start 146.8031 91.378) (end 145.9851 90.56) (width 0.3) (layer "F.Cu") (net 26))
 (segment (start 152.135 91.378) (end 146.8031 91.378) (width 0.3) (layer "F.Cu") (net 26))
 (segment (start 142.2319 91.383) (end 143.0499 90.565) (width 0.3) (layer "F.Cu") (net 17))
 (segment (start 136.9 91.383) (end 142.2319 91.383) (width 0.3) (layer "F.Cu") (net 17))
 (segment (start 143.875 90.565) (end 143.0499 90.565) (width 0.3) (layer "F.Cu") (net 17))
 (segment (start 152.135 93.156) (end 147.3111 93.156) (width 0.3) (layer "F.Cu") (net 25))
 (segment (start 145.16 91.83) (end 145.9851 91.83) (width 0.3) (layer "F.Cu") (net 25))
 (segment (start 147.3111 93.156) (end 145.9851 91.83) (width 0.3) (layer "F.Cu") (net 25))
 (segment (start 143.875 91.835) (end 143.0499 91.835) (width 0.3) (layer "F.Cu") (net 18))
 (segment (start 141.7239 93.161) (end 143.0499 91.835) (width 0.3) (layer "F.Cu") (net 18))
 (segment (start 136.9 93.161) (end 141.7239 93.161) (width 0.3) (layer "F.Cu") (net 18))
 (segment (start 145.16 93.1) (end 145.9851 93.1) (width 0.3) (layer "F.Cu") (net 24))
 (segment (start 147.8191 94.934) (end 145.9851 93.1) (width 0.3) (layer "F.Cu") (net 24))
 (segment (start 152.135 94.934) (end 147.8191 94.934) (width 0.3) (layer "F.Cu") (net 24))
 (segment (start 143.875 93.105) (end 143.0499 93.105) (width 0.3) (layer "F.Cu") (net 19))
 (segment (start 141.2159 94.939) (end 143.0499 93.105) (width 0.3) (layer "F.Cu") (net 19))
 (segment (start 136.9 94.939) (end 141.2159 94.939) (width 0.3) (layer "F.Cu") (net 19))
 (segment (start 148.3271 96.712) (end 145.9851 94.37) (width 0.3) (layer "F.Cu") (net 23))
 (segment (start 152.135 96.712) (end 148.3271 96.712) (width 0.3) (layer "F.Cu") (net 23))
 (segment (start 145.16 94.37) (end 145.9851 94.37) (width 0.3) (layer "F.Cu") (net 23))
 (segment (start 136.9 96.717) (end 140.7079 96.717) (width 0.3) (layer "F.Cu") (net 20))
 (segment (start 140.7079 96.717) (end 143.0499 94.375) (width 0.3) (layer "F.Cu") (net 20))
 (segment (start 143.875 94.375) (end 143.0499 94.375) (width 0.3) (layer "F.Cu") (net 20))
 (segment (start 145.16 95.64) (end 145.9851 95.64) (width 0.3) (layer "F.Cu") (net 22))
 (segment (start 152.135 98.49) (end 148.8351 98.49) (width 0.3) (layer "F.Cu") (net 22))
 (segment (start 148.8351 98.49) (end 145.9851 95.64) (width 0.3) (layer "F.Cu") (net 22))
 (segment (start 143.875 95.645) (end 143.0499 95.645) (width 0.3) (layer "F.Cu") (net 21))
 (segment (start 136.9 98.495) (end 140.1999 98.495) (width 0.3) (layer "F.Cu") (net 21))
 (segment (start 140.1999 98.495) (end 143.0499 95.645) (width 0.3) (layer "F.Cu") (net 21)))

